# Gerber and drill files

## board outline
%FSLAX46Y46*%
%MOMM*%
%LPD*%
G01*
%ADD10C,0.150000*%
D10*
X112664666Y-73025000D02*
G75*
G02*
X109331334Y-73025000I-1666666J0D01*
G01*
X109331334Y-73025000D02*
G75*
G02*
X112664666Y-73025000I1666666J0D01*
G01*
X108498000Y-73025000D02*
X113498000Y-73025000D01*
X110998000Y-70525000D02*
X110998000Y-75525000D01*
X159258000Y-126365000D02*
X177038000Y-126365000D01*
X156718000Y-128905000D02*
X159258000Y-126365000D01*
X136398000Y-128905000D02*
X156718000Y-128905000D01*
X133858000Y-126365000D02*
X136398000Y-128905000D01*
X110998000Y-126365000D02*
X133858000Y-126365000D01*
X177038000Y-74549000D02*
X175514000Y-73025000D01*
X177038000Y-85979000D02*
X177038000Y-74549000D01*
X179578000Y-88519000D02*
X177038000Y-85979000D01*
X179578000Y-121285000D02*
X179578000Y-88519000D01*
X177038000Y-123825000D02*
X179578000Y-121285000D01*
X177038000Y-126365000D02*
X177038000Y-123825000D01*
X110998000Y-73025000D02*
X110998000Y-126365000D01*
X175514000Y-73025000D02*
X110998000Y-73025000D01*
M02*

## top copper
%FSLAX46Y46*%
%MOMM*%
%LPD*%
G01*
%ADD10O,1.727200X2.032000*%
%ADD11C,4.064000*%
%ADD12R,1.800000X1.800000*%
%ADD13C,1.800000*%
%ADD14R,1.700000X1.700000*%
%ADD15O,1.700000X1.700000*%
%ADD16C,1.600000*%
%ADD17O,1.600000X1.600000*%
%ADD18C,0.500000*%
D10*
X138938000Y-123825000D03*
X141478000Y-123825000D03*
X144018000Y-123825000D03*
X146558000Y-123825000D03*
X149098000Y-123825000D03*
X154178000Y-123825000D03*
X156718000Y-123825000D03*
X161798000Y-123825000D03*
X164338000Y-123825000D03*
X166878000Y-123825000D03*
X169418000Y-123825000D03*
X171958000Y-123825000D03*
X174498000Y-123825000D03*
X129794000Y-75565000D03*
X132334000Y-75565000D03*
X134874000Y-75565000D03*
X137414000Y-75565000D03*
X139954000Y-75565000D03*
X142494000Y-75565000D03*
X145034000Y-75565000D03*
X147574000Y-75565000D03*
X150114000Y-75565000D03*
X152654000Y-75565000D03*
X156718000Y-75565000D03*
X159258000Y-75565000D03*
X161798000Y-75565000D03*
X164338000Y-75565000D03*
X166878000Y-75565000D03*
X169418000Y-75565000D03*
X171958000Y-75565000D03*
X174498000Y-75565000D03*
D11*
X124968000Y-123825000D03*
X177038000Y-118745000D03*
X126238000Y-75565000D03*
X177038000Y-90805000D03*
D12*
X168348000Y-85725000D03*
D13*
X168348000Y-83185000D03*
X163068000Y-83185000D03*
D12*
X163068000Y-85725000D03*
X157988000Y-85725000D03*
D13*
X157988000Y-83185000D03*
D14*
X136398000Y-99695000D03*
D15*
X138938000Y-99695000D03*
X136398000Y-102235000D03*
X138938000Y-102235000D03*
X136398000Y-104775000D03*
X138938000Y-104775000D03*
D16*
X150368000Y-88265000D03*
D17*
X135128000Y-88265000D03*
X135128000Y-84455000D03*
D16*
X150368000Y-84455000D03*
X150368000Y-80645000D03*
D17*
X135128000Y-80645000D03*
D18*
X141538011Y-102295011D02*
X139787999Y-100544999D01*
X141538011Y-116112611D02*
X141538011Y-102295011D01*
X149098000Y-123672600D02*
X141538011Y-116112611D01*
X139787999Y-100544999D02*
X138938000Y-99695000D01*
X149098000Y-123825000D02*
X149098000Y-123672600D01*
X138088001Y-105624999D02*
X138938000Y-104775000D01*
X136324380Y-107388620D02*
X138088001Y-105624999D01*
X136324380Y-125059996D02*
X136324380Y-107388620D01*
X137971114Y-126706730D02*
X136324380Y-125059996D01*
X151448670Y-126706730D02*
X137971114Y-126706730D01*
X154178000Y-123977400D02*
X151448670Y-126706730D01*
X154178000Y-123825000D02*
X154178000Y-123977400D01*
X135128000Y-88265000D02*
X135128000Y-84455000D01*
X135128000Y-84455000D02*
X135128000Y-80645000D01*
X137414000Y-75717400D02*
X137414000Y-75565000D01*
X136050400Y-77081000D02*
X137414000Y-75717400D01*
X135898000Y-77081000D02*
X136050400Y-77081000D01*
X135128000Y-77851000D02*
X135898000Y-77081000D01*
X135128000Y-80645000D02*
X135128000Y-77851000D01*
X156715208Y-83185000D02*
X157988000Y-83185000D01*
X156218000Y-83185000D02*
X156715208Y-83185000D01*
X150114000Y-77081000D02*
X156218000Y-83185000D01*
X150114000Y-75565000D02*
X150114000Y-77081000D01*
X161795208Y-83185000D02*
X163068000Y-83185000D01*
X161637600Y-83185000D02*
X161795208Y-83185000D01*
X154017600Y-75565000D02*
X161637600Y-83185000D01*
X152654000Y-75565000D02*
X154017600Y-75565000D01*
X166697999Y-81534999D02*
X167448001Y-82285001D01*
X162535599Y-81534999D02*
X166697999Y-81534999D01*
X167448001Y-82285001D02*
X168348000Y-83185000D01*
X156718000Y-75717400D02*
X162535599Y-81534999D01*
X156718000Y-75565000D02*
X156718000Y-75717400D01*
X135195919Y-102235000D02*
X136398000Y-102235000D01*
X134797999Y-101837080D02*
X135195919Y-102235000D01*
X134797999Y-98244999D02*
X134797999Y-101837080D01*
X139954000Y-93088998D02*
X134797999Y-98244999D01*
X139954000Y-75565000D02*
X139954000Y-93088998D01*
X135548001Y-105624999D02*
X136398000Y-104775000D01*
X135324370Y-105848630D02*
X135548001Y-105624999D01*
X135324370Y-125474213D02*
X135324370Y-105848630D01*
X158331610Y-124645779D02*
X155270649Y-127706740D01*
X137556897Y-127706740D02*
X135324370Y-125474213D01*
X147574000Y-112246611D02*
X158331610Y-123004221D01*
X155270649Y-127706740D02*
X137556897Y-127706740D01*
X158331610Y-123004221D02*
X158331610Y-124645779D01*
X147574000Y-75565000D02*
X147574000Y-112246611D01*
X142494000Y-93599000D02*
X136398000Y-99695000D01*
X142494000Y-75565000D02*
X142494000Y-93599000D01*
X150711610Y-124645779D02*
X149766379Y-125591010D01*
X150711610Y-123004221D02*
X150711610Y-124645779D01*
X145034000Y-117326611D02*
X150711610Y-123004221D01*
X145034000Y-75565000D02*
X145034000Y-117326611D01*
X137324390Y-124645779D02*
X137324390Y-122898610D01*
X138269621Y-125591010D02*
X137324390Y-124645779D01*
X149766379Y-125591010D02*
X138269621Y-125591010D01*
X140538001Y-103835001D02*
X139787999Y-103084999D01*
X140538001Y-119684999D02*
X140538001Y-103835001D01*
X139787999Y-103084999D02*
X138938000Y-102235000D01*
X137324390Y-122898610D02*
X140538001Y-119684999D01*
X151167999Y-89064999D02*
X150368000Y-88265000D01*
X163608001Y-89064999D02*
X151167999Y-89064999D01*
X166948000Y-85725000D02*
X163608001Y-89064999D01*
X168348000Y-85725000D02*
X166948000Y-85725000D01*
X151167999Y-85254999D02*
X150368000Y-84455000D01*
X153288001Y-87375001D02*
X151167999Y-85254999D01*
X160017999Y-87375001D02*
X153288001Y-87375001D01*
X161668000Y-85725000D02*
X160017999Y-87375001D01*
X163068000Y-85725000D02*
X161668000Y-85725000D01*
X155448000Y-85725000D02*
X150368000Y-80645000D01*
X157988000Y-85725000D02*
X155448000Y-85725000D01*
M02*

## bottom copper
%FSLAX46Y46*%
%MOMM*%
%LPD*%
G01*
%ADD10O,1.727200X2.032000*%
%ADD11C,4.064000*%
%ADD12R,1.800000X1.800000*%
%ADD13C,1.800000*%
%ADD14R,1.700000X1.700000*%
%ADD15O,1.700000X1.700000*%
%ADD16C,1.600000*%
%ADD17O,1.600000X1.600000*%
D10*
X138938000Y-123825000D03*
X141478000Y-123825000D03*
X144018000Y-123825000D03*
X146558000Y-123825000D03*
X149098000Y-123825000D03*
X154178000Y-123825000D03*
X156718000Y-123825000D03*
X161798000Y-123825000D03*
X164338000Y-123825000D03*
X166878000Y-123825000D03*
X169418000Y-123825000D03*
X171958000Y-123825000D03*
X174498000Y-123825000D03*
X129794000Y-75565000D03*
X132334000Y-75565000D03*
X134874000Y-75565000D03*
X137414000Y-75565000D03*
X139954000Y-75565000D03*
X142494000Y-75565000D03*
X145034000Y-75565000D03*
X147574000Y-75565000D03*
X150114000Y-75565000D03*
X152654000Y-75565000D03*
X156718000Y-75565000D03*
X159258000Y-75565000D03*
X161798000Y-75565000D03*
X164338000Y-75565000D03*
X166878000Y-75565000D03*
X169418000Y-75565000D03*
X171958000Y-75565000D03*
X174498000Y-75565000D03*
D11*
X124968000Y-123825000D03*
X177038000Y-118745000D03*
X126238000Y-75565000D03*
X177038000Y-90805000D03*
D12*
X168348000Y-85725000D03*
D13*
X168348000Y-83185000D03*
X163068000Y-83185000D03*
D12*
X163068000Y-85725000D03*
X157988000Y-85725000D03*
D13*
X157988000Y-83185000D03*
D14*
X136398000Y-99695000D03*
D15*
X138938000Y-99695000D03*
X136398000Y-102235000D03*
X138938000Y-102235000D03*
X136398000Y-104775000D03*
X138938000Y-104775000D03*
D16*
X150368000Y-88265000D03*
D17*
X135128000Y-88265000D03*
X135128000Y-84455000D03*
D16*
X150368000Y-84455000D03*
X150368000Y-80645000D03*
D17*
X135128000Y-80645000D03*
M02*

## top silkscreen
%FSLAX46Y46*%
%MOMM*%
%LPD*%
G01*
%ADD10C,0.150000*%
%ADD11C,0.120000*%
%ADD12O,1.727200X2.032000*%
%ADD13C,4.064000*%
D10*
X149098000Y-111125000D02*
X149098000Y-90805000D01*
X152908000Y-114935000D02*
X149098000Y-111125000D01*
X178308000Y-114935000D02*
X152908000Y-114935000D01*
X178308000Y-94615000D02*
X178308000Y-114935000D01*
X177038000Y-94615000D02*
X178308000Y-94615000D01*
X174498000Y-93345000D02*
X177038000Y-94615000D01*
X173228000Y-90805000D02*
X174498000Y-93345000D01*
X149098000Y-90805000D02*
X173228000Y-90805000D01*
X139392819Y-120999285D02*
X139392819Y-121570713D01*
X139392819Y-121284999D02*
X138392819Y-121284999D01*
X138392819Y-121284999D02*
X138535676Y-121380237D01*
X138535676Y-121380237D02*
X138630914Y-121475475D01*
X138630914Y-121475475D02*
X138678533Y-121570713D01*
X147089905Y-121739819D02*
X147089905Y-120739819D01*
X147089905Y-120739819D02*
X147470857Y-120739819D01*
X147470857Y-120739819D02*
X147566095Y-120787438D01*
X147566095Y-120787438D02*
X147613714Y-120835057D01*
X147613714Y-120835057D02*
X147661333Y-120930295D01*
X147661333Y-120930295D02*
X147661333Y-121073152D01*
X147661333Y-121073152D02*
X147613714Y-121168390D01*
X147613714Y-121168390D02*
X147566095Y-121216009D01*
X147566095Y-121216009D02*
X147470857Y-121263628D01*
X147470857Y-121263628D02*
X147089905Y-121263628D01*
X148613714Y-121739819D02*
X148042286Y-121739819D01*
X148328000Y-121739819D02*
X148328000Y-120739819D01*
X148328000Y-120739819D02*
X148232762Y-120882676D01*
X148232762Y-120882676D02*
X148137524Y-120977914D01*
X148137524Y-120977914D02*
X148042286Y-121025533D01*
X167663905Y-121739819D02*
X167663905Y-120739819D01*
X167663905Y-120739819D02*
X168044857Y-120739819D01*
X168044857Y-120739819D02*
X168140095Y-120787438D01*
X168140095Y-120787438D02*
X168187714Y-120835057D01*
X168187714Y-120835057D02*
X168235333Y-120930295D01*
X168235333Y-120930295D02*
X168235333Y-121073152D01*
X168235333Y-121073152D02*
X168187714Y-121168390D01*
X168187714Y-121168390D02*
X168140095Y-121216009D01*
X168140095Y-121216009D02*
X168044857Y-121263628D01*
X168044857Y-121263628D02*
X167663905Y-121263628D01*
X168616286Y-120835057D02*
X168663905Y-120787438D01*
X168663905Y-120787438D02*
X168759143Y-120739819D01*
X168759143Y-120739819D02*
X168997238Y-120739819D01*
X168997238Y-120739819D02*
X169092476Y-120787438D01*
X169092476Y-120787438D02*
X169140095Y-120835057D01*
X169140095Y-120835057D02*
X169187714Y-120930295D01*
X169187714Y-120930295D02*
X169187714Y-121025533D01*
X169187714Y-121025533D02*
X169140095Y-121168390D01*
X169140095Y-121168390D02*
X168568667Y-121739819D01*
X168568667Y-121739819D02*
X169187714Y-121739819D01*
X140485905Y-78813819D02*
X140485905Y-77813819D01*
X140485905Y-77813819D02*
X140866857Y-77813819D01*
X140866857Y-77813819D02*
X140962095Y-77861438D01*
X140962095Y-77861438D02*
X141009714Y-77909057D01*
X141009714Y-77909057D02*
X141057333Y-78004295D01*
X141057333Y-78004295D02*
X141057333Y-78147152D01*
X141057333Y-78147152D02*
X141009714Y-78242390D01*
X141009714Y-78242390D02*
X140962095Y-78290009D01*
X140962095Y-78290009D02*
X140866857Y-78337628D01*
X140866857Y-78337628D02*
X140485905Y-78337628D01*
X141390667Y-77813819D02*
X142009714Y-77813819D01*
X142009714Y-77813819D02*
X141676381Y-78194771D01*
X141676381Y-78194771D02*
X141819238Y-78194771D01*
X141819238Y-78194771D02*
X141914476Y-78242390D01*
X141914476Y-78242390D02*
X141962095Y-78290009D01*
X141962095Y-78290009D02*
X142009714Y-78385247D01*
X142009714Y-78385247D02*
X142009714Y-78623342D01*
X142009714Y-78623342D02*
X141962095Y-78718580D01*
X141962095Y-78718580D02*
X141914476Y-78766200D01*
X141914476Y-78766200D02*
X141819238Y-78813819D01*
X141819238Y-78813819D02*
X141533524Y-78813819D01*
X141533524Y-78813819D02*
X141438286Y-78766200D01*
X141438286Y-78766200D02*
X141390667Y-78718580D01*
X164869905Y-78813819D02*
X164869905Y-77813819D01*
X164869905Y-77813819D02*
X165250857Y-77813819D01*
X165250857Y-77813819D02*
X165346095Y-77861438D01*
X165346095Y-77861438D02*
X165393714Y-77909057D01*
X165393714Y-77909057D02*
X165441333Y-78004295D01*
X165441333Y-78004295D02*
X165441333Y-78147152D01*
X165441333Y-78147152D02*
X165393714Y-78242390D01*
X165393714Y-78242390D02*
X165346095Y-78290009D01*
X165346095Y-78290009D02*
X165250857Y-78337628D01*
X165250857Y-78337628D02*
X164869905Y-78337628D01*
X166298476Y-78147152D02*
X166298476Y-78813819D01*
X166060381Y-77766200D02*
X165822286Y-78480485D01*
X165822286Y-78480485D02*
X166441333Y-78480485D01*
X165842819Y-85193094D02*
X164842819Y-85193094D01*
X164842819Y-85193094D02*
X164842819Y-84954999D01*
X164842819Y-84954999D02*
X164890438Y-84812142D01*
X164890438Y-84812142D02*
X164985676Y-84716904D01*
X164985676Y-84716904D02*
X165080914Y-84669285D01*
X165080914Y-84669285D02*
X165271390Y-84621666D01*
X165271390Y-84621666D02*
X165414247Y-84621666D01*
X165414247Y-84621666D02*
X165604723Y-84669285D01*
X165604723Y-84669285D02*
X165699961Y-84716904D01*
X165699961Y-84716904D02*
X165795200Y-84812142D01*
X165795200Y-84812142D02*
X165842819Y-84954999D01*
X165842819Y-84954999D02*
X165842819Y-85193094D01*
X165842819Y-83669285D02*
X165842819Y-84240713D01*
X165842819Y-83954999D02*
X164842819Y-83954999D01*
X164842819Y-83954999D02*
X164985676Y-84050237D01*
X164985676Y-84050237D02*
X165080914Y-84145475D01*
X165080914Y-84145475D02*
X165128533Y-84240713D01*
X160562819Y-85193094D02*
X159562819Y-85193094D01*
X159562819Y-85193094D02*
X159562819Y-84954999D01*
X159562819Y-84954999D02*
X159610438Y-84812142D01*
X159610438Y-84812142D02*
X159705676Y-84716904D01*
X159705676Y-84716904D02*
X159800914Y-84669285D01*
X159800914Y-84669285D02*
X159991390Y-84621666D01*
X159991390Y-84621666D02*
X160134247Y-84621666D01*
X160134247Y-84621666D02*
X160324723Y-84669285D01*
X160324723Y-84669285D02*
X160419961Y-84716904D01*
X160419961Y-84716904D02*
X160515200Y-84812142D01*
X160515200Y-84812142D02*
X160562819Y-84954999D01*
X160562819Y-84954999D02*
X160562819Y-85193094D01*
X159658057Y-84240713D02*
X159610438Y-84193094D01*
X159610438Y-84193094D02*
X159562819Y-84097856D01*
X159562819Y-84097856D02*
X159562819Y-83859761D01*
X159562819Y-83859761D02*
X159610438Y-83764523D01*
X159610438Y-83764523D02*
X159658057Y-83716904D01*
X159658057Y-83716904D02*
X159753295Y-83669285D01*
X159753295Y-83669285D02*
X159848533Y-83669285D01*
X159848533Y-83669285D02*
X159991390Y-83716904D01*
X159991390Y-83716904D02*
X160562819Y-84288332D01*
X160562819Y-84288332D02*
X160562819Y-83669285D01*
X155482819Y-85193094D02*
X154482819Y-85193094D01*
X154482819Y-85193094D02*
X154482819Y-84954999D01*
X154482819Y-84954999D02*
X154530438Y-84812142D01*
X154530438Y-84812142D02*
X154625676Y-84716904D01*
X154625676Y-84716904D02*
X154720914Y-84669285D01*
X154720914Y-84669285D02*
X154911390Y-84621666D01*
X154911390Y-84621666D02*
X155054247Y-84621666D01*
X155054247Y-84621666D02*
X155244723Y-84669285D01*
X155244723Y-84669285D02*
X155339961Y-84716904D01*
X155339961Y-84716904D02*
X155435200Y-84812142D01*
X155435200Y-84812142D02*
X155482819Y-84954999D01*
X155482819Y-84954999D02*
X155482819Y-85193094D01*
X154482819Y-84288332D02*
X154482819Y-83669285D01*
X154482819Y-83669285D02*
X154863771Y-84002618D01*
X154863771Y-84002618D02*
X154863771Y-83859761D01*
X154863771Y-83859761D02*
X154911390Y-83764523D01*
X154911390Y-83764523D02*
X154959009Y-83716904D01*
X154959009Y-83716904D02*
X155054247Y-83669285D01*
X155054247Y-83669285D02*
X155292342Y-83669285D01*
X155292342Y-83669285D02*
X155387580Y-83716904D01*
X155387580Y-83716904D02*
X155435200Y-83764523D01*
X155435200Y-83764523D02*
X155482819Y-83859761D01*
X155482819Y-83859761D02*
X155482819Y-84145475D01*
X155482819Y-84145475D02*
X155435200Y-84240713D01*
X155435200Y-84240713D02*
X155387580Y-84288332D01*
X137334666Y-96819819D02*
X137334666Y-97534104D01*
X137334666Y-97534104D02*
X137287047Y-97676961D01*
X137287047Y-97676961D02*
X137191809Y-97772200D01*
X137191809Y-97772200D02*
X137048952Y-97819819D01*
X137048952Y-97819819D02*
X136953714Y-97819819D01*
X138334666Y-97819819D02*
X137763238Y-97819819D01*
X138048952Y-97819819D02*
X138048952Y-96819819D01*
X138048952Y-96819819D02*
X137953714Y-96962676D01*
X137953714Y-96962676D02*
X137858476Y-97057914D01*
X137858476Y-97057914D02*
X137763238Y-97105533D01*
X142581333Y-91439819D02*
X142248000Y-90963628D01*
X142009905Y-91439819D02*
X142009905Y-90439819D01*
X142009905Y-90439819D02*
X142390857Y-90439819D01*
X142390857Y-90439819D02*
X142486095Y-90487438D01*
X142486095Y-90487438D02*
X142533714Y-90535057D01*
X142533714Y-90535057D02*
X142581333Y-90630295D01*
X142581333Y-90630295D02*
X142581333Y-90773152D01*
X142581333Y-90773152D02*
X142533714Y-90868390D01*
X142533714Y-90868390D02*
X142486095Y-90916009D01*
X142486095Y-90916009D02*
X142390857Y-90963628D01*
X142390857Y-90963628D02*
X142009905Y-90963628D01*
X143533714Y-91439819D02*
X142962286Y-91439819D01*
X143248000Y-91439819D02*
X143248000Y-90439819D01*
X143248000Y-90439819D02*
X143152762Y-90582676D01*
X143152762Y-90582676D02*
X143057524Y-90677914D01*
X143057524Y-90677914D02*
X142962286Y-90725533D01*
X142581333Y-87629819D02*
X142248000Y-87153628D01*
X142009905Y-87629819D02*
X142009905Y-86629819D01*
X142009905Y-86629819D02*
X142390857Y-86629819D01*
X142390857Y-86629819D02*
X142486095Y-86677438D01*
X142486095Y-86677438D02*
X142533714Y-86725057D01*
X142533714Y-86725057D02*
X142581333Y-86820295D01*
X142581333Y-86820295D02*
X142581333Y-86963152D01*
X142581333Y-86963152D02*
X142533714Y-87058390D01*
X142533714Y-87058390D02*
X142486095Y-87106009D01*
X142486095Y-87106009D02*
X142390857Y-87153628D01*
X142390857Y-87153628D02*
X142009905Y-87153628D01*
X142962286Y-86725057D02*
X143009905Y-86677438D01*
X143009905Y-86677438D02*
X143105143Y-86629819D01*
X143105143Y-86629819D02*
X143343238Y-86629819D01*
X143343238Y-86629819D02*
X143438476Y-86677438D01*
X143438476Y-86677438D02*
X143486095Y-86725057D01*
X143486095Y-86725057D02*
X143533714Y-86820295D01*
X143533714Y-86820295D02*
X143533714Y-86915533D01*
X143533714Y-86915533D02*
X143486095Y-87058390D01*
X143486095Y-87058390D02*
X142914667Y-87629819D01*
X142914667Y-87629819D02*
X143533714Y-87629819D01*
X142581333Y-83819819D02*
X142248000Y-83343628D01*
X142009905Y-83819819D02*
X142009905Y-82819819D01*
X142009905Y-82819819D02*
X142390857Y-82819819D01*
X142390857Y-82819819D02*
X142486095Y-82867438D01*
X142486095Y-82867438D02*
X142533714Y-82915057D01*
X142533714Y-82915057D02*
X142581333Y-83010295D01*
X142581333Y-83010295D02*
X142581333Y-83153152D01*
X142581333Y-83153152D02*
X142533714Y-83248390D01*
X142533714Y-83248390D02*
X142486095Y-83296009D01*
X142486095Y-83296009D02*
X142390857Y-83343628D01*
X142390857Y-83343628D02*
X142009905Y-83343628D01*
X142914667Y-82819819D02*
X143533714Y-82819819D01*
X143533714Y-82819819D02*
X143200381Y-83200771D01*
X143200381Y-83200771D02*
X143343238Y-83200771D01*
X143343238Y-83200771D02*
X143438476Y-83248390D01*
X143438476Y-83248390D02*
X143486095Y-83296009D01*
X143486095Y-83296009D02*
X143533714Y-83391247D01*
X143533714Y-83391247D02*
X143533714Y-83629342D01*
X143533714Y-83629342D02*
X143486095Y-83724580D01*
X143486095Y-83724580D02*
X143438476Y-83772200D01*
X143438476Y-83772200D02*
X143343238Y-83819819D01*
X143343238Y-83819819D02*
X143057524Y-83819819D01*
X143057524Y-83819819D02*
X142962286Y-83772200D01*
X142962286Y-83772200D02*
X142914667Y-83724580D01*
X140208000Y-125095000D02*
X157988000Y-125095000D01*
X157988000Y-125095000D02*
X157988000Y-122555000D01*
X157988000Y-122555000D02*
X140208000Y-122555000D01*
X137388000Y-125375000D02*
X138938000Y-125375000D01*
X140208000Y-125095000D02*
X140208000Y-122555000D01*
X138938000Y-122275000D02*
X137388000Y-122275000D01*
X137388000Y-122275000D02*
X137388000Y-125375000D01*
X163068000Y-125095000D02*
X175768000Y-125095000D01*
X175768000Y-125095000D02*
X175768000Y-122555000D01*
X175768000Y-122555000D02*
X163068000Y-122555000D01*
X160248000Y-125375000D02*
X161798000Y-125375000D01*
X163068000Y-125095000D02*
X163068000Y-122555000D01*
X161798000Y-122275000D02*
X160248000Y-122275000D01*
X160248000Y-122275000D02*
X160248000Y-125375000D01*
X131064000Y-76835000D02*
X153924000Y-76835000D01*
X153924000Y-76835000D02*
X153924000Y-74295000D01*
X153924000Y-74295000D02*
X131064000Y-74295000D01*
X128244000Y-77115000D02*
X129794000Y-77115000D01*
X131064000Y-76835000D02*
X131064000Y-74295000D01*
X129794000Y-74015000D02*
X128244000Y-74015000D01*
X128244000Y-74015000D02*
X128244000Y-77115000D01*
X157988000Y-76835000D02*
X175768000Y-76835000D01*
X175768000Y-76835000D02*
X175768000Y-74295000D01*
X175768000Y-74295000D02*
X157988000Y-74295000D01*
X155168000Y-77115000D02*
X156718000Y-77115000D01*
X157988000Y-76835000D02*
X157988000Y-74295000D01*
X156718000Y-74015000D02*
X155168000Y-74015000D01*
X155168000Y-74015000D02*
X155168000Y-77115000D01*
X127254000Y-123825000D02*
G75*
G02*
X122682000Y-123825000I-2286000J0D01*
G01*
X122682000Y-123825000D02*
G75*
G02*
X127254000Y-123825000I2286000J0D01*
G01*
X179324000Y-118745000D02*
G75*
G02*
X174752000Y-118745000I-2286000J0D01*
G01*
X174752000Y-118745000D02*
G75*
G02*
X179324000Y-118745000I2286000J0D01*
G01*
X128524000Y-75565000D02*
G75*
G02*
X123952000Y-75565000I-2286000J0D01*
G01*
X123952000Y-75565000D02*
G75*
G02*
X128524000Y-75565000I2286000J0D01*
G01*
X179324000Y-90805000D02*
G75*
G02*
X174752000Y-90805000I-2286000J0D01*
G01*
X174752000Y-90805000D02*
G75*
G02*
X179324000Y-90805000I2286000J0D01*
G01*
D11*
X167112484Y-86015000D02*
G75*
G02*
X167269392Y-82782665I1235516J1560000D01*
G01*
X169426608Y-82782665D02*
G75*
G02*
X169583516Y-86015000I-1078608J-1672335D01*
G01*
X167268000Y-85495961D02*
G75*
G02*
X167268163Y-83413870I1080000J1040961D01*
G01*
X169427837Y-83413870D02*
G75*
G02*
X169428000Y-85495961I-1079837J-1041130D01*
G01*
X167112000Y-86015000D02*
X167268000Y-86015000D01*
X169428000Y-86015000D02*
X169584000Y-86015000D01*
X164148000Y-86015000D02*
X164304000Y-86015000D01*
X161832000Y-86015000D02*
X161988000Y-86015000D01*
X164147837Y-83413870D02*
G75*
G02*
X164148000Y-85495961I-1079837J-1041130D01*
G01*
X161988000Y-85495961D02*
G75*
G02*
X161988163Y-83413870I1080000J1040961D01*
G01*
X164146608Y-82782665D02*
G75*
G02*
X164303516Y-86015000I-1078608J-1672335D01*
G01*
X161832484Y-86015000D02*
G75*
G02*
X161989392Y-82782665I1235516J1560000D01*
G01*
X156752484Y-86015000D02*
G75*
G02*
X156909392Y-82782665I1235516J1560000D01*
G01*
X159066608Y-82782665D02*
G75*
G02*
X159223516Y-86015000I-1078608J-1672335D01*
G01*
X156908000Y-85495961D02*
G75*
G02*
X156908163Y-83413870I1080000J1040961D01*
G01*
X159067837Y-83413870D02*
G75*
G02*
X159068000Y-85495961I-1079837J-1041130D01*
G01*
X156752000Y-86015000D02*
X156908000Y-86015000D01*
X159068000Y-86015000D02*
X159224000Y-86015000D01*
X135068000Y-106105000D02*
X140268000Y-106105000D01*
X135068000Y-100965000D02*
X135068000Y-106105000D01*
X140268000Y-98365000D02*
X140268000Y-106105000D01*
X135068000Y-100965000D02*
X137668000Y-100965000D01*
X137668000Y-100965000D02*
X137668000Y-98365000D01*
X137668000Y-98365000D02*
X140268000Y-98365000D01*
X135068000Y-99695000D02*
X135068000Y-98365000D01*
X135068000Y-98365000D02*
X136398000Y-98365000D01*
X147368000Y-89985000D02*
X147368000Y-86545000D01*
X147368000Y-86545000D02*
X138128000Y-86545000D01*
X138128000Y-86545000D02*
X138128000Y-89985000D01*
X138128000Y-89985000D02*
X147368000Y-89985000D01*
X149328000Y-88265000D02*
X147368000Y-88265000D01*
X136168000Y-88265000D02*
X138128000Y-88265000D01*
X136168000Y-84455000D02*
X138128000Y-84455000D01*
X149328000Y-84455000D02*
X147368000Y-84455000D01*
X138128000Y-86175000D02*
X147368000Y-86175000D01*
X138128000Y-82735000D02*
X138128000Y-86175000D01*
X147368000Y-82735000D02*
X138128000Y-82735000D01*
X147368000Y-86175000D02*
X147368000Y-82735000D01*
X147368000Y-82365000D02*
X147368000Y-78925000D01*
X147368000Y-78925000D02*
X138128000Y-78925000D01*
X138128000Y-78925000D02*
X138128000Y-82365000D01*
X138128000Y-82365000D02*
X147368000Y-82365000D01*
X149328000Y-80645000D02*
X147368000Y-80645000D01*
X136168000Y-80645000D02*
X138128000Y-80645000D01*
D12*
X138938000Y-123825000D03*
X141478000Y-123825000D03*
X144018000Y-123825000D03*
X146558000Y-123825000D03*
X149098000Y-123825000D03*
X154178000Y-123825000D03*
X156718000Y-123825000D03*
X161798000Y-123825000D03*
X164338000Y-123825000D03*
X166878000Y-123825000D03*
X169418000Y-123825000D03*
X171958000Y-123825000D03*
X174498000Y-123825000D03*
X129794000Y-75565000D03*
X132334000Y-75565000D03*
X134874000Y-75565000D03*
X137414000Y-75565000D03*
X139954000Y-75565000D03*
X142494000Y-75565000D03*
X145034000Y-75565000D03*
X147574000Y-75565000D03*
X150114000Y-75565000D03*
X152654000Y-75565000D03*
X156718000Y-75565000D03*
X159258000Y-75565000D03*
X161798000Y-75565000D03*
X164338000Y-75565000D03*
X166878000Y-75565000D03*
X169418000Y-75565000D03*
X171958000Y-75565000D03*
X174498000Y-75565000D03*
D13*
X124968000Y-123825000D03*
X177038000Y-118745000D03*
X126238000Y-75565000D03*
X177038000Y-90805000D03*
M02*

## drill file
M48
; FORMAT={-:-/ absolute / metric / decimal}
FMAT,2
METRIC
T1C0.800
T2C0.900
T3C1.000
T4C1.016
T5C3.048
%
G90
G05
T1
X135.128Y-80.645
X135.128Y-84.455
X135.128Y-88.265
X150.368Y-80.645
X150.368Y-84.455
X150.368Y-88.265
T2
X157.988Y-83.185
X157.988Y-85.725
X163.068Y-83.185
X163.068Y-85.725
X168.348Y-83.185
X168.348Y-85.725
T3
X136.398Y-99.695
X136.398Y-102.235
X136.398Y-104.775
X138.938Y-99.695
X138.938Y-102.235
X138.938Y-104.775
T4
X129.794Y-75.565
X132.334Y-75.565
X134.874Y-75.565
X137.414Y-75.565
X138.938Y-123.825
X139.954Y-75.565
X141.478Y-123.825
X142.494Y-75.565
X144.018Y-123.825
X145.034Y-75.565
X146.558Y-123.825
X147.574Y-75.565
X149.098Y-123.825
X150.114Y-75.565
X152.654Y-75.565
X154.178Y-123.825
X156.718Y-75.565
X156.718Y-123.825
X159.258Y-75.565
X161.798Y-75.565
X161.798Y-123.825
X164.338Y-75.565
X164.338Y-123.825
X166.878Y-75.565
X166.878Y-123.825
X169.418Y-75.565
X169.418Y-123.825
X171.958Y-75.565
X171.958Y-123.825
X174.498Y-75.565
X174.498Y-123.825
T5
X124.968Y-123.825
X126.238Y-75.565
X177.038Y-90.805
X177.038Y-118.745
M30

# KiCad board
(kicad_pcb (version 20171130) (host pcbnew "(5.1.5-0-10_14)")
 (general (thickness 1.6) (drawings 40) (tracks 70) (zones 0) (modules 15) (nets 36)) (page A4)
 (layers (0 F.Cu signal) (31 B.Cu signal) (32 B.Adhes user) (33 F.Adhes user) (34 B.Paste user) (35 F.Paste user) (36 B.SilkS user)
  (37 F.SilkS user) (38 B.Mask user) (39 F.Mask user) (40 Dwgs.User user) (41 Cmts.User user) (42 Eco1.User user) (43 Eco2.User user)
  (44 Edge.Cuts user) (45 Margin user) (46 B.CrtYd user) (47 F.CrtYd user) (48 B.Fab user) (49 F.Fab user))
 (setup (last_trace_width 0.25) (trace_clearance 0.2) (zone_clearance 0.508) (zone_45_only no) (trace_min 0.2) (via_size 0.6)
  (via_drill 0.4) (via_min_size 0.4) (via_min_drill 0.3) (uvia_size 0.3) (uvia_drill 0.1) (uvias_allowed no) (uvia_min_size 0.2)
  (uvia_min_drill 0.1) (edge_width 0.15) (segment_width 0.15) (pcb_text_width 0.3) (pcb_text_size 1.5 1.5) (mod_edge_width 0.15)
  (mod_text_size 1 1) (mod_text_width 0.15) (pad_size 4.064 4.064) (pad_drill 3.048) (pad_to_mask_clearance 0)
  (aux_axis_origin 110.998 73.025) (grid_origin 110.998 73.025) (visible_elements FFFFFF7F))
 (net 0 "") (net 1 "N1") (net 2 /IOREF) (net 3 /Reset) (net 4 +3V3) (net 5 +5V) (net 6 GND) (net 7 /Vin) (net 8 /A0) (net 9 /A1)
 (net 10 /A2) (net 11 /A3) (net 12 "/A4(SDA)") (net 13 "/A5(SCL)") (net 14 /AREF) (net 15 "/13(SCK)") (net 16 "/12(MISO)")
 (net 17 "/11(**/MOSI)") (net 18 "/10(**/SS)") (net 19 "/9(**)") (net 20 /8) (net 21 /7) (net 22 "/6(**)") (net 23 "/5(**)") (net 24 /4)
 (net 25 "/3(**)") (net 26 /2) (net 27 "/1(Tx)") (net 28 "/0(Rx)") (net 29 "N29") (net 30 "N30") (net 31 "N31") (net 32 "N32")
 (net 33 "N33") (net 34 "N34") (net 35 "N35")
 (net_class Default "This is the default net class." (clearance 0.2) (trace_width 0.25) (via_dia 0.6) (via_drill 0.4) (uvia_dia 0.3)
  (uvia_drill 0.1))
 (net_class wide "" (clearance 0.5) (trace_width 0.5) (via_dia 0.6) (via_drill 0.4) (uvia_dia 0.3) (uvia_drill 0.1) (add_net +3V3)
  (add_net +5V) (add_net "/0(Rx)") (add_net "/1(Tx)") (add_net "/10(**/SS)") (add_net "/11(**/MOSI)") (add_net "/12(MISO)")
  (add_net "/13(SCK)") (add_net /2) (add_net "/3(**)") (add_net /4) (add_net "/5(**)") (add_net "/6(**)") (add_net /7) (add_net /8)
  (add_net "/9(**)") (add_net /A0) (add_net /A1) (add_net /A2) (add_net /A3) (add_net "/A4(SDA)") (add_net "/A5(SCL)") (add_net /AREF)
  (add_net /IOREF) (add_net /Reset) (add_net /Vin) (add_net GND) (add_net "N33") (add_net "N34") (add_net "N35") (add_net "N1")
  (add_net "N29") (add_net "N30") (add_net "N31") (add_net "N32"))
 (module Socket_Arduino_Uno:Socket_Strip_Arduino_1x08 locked (layer F.Cu) (at 138.938 123.825)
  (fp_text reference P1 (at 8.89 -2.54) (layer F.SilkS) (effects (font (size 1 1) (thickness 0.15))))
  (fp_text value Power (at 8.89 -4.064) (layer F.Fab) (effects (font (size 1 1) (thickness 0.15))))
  (fp_line (start 1.27 1.27) (end 19.05 1.27) (layer F.SilkS) (width 0.15))
  (fp_line (start 19.05 1.27) (end 19.05 -1.27) (layer F.SilkS) (width 0.15))
  (fp_line (start 19.05 -1.27) (end 1.27 -1.27) (layer F.SilkS) (width 0.15))
  (fp_line (start -1.55 1.55) (end 0 1.55) (layer F.SilkS) (width 0.15))
  (fp_line (start 1.27 1.27) (end 1.27 -1.27) (layer F.SilkS) (width 0.15))
  (fp_line (start 0 -1.55) (end -1.55 -1.55) (layer F.SilkS) (width 0.15))
  (fp_line (start -1.55 -1.55) (end -1.55 1.55) (layer F.SilkS) (width 0.15))
  (pad 1 thru_hole oval (at 0 0) (size 1.7272 2.032) (drill 1.016) (layers *.Cu *.Mask F.SilkS) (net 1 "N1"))
  (pad 2 thru_hole oval (at 2.54 0) (size 1.7272 2.032) (drill 1.016) (layers *.Cu *.Mask F.SilkS) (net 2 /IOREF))
  (pad 3 thru_hole oval (at 5.08 0) (size 1.7272 2.032) (drill 1.016) (layers *.Cu *.Mask F.SilkS) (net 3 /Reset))
  (pad 4 thru_hole oval (at 7.62 0) (size 1.7272 2.032) (drill 1.016) (layers *.Cu *.Mask F.SilkS) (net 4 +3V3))
  (pad 5 thru_hole oval (at 10.16 0) (size 1.7272 2.032) (drill 1.016) (layers *.Cu *.Mask F.SilkS) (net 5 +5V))
  (pad 6 connect oval (at 12.7 0) (size 1.7272 2.032) (layers Dwgs.User) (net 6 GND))
  (pad 7 thru_hole oval (at 15.24 0) (size 1.7272 2.032) (drill 1.016) (layers *.Cu *.Mask F.SilkS) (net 6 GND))
  (pad 8 thru_hole oval (at 17.78 0) (size 1.7272 2.032) (drill 1.016) (layers *.Cu *.Mask F.SilkS) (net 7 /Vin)))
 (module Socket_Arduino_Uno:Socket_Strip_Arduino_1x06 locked (layer F.Cu) (at 161.798 123.825)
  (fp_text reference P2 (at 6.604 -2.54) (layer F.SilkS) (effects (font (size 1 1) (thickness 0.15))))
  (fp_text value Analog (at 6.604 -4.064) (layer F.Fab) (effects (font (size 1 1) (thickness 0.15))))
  (fp_line (start 1.27 1.27) (end 13.97 1.27) (layer F.SilkS) (width 0.15))
  (fp_line (start 13.97 1.27) (end 13.97 -1.27) (layer F.SilkS) (width 0.15))
  (fp_line (start 13.97 -1.27) (end 1.27 -1.27) (layer F.SilkS) (width 0.15))
  (fp_line (start -1.55 1.55) (end 0 1.55) (layer F.SilkS) (width 0.15))
  (fp_line (start 1.27 1.27) (end 1.27 -1.27) (layer F.SilkS) (width 0.15))
  (fp_line (start 0 -1.55) (end -1.55 -1.55) (layer F.SilkS) (width 0.15))
  (fp_line (start -1.55 -1.55) (end -1.55 1.55) (layer F.SilkS) (width 0.15))
  (pad 1 thru_hole oval (at 0 0) (size 1.7272 2.032) (drill 1.016) (layers *.Cu *.Mask F.SilkS) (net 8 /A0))
  (pad 2 thru_hole oval (at 2.54 0) (size 1.7272 2.032) (drill 1.016) (layers *.Cu *.Mask F.SilkS) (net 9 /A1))
  (pad 3 thru_hole oval (at 5.08 0) (size 1.7272 2.032) (drill 1.016) (layers *.Cu *.Mask F.SilkS) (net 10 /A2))
  (pad 4 thru_hole oval (at 7.62 0) (size 1.7272 2.032) (drill 1.016) (layers *.Cu *.Mask F.SilkS) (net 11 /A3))
  (pad 5 thru_hole oval (at 10.16 0) (size 1.7272 2.032) (drill 1.016) (layers *.Cu *.Mask F.SilkS) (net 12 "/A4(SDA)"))
  (pad 6 thru_hole oval (at 12.7 0) (size 1.7272 2.032) (drill 1.016) (layers *.Cu *.Mask F.SilkS) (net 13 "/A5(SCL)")))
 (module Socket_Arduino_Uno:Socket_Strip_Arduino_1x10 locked (layer F.Cu) (at 129.794 75.565)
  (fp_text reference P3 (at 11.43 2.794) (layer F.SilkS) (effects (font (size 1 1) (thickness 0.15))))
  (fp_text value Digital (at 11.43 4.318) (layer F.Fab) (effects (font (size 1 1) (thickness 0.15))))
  (fp_line (start 1.27 1.27) (end 24.13 1.27) (layer F.SilkS) (width 0.15))
  (fp_line (start 24.13 1.27) (end 24.13 -1.27) (layer F.SilkS) (width 0.15))
  (fp_line (start 24.13 -1.27) (end 1.27 -1.27) (layer F.SilkS) (width 0.15))
  (fp_line (start -1.55 1.55) (end 0 1.55) (layer F.SilkS) (width 0.15))
  (fp_line (start 1.27 1.27) (end 1.27 -1.27) (layer F.SilkS) (width 0.15))
  (fp_line (start 0 -1.55) (end -1.55 -1.55) (layer F.SilkS) (width 0.15))
  (fp_line (start -1.55 -1.55) (end -1.55 1.55) (layer F.SilkS) (width 0.15))
  (pad 1 thru_hole oval (at 0 0) (size 1.7272 2.032) (drill 1.016) (layers *.Cu *.Mask F.SilkS) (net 13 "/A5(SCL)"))
  (pad 2 thru_hole oval (at 2.54 0) (size 1.7272 2.032) (drill 1.016) (layers *.Cu *.Mask F.SilkS) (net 12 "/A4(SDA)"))
  (pad 3 thru_hole oval (at 5.08 0) (size 1.7272 2.032) (drill 1.016) (layers *.Cu *.Mask F.SilkS) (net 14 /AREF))
  (pad 4 thru_hole oval (at 7.62 0) (size 1.7272 2.032) (drill 1.016) (layers *.Cu *.Mask F.SilkS) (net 6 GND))
  (pad 5 thru_hole oval (at 10.16 0) (size 1.7272 2.032) (drill 1.016) (layers *.Cu *.Mask F.SilkS) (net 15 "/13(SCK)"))
  (pad 6 thru_hole oval (at 12.7 0) (size 1.7272 2.032) (drill 1.016) (layers *.Cu *.Mask F.SilkS) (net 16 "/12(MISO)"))
  (pad 7 thru_hole oval (at 15.24 0) (size 1.7272 2.032) (drill 1.016) (layers *.Cu *.Mask F.SilkS) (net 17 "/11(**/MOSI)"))
  (pad 8 thru_hole oval (at 17.78 0) (size 1.7272 2.032) (drill 1.016) (layers *.Cu *.Mask F.SilkS) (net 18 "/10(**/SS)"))
  (pad 9 thru_hole oval (at 20.32 0) (size 1.7272 2.032) (drill 1.016) (layers *.Cu *.Mask F.SilkS) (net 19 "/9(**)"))
  (pad 10 thru_hole oval (at 22.86 0) (size 1.7272 2.032) (drill 1.016) (layers *.Cu *.Mask F.SilkS) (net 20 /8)))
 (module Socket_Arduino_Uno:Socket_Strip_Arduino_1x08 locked (layer F.Cu) (at 156.718 75.565)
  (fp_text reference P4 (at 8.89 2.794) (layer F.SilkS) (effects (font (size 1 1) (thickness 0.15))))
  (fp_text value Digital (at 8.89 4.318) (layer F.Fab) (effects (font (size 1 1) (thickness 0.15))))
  (fp_line (start 1.27 1.27) (end 19.05 1.27) (layer F.SilkS) (width 0.15))
  (fp_line (start 19.05 1.27) (end 19.05 -1.27) (layer F.SilkS) (width 0.15))
  (fp_line (start 19.05 -1.27) (end 1.27 -1.27) (layer F.SilkS) (width 0.15))
  (fp_line (start -1.55 1.55) (end 0 1.55) (layer F.SilkS) (width 0.15))
  (fp_line (start 1.27 1.27) (end 1.27 -1.27) (layer F.SilkS) (width 0.15))
  (fp_line (start 0 -1.55) (end -1.55 -1.55) (layer F.SilkS) (width 0.15))
  (fp_line (start -1.55 -1.55) (end -1.55 1.55) (layer F.SilkS) (width 0.15))
  (pad 1 thru_hole oval (at 0 0) (size 1.7272 2.032) (drill 1.016) (layers *.Cu *.Mask F.SilkS) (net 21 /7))
  (pad 2 thru_hole oval (at 2.54 0) (size 1.7272 2.032) (drill 1.016) (layers *.Cu *.Mask F.SilkS) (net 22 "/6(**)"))
  (pad 3 thru_hole oval (at 5.08 0) (size 1.7272 2.032) (drill 1.016) (layers *.Cu *.Mask F.SilkS) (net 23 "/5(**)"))
  (pad 4 thru_hole oval (at 7.62 0) (size 1.7272 2.032) (drill 1.016) (layers *.Cu *.Mask F.SilkS) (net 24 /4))
  (pad 5 thru_hole oval (at 10.16 0) (size 1.7272 2.032) (drill 1.016) (layers *.Cu *.Mask F.SilkS) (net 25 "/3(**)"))
  (pad 6 thru_hole oval (at 12.7 0) (size 1.7272 2.032) (drill 1.016) (layers *.Cu *.Mask F.SilkS) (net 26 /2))
  (pad 7 thru_hole oval (at 15.24 0) (size 1.7272 2.032) (drill 1.016) (layers *.Cu *.Mask F.SilkS) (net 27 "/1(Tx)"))
  (pad 8 thru_hole oval (at 17.78 0) (size 1.7272 2.032) (drill 1.016) (layers *.Cu *.Mask F.SilkS) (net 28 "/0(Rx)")))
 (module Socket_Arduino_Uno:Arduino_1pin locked (layer F.Cu) (at 124.968 123.825)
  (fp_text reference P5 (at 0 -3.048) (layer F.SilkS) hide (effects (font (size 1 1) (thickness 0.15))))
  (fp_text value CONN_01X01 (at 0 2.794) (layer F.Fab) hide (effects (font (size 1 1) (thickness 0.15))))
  (fp_circle (center 0 0) (end 0 -2.286) (layer F.SilkS) (width 0.15))
  (pad 1 thru_hole circle (at 0 0) (size 4.064 4.064) (drill 3.048) (layers *.Cu *.Mask F.SilkS) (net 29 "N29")))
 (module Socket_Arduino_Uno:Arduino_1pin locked (layer F.Cu) (at 177.038 118.745)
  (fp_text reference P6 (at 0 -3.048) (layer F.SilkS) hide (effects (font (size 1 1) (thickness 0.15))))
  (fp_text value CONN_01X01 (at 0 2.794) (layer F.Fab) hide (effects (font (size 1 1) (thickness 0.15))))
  (fp_circle (center 0 0) (end 0 -2.286) (layer F.SilkS) (width 0.15))
  (pad 1 thru_hole circle (at 0 0) (size 4.064 4.064) (drill 3.048) (layers *.Cu *.Mask F.SilkS) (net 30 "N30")))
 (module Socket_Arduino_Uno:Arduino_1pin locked (layer F.Cu) (at 126.238 75.565)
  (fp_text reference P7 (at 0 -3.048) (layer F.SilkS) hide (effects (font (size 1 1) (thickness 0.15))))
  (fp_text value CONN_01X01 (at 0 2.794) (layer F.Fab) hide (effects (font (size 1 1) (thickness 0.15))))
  (fp_circle (center 0 0) (end 0 -2.286) (layer F.SilkS) (width 0.15))
  (pad 1 thru_hole circle (at 0 0) (size 4.064 4.064) (drill 3.048) (layers *.Cu *.Mask F.SilkS) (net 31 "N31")))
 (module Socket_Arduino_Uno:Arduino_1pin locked (layer F.Cu) (at 177.038 90.805)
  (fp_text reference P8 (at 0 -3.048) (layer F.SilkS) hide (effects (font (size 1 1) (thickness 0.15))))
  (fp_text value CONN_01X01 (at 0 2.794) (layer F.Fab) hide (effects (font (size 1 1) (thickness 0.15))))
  (fp_circle (center 0 0) (end 0 -2.286) (layer F.SilkS) (width 0.15))
  (pad 1 thru_hole circle (at 0 0) (size 4.064 4.064) (drill 3.048) (layers *.Cu *.Mask F.SilkS) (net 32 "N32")))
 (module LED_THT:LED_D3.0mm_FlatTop (layer F.Cu) (at 168.348 85.725 90)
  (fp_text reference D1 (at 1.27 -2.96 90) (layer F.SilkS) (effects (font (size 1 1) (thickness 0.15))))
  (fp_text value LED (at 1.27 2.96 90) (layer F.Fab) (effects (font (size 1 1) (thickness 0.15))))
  (fp_arc (start 1.27 0) (end -0.29 -1.235516) (angle 108.8) (layer F.SilkS) (width 0.12))
  (fp_arc (start 1.27 0) (end -0.29 1.235516) (angle -108.8) (layer F.SilkS) (width 0.12))
  (fp_arc (start 1.27 0) (end 0.229039 -1.08) (angle 87.9) (layer F.SilkS) (width 0.12))
  (fp_arc (start 1.27 0) (end 0.229039 1.08) (angle -87.9) (layer F.SilkS) (width 0.12))
  (fp_line (start -0.29 -1.236) (end -0.29 -1.08) (layer F.SilkS) (width 0.12))
  (fp_line (start -0.29 1.08) (end -0.29 1.236) (layer F.SilkS) (width 0.12))
  (pad 1 thru_hole rect (at 0 0 90) (size 1.8 1.8) (drill 0.9) (layers *.Cu *.Mask) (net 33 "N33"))
  (pad 2 thru_hole circle (at 2.54 0 90) (size 1.8 1.8) (drill 0.9) (layers *.Cu *.Mask) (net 21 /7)))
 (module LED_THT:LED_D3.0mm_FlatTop (layer F.Cu) (at 163.068 85.725 90)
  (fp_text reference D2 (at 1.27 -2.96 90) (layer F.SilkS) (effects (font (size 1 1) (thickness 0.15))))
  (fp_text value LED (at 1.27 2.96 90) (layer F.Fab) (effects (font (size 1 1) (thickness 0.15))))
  (fp_line (start -0.29 1.08) (end -0.29 1.236) (layer F.SilkS) (width 0.12))
  (fp_line (start -0.29 -1.236) (end -0.29 -1.08) (layer F.SilkS) (width 0.12))
  (fp_arc (start 1.27 0) (end 0.229039 1.08) (angle -87.9) (layer F.SilkS) (width 0.12))
  (fp_arc (start 1.27 0) (end 0.229039 -1.08) (angle 87.9) (layer F.SilkS) (width 0.12))
  (fp_arc (start 1.27 0) (end -0.29 1.235516) (angle -108.8) (layer F.SilkS) (width 0.12))
  (fp_arc (start 1.27 0) (end -0.29 -1.235516) (angle 108.8) (layer F.SilkS) (width 0.12))
  (pad 2 thru_hole circle (at 2.54 0 90) (size 1.8 1.8) (drill 0.9) (layers *.Cu *.Mask) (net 20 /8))
  (pad 1 thru_hole rect (at 0 0 90) (size 1.8 1.8) (drill 0.9) (layers *.Cu *.Mask) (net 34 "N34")))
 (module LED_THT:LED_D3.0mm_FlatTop (layer F.Cu) (at 157.988 85.725 90)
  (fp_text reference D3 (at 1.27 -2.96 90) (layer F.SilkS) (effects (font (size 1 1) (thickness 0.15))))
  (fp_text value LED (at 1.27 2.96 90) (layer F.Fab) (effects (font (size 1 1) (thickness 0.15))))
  (fp_arc (start 1.27 0) (end -0.29 -1.235516) (angle 108.8) (layer F.SilkS) (width 0.12))
  (fp_arc (start 1.27 0) (end -0.29 1.235516) (angle -108.8) (layer F.SilkS) (width 0.12))
  (fp_arc (start 1.27 0) (end 0.229039 -1.08) (angle 87.9) (layer F.SilkS) (width 0.12))
  (fp_arc (start 1.27 0) (end 0.229039 1.08) (angle -87.9) (layer F.SilkS) (width 0.12))
  (fp_line (start -0.29 -1.236) (end -0.29 -1.08) (layer F.SilkS) (width 0.12))
  (fp_line (start -0.29 1.08) (end -0.29 1.236) (layer F.SilkS) (width 0.12))
  (pad 1 thru_hole rect (at 0 0 90) (size 1.8 1.8) (drill 0.9) (layers *.Cu *.Mask) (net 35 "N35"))
  (pad 2 thru_hole circle (at 2.54 0 90) (size 1.8 1.8) (drill 0.9) (layers *.Cu *.Mask) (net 19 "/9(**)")))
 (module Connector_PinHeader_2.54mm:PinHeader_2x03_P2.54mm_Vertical (layer F.Cu) (at 136.398 99.695)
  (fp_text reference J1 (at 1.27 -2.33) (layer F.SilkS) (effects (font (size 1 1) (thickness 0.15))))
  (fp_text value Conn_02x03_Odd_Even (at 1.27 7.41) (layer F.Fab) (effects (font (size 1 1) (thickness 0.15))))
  (fp_line (start -1.33 6.41) (end 3.87 6.41) (layer F.SilkS) (width 0.12))
  (fp_line (start -1.33 1.27) (end -1.33 6.41) (layer F.SilkS) (width 0.12))
  (fp_line (start 3.87 -1.33) (end 3.87 6.41) (layer F.SilkS) (width 0.12))
  (fp_line (start -1.33 1.27) (end 1.27 1.27) (layer F.SilkS) (width 0.12))
  (fp_line (start 1.27 1.27) (end 1.27 -1.33) (layer F.SilkS) (width 0.12))
  (fp_line (start 1.27 -1.33) (end 3.87 -1.33) (layer F.SilkS) (width 0.12))
  (fp_line (start -1.33 0) (end -1.33 -1.33) (layer F.SilkS) (width 0.12))
  (fp_line (start -1.33 -1.33) (end 0 -1.33) (layer F.SilkS) (width 0.12))
  (pad 1 thru_hole rect (at 0 0) (size 1.7 1.7) (drill 1) (layers *.Cu *.Mask) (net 16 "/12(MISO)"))
  (pad 2 thru_hole oval (at 2.54 0) (size 1.7 1.7) (drill 1) (layers *.Cu *.Mask) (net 5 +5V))
  (pad 3 thru_hole oval (at 0 2.54) (size 1.7 1.7) (drill 1) (layers *.Cu *.Mask) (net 15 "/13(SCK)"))
  (pad 4 thru_hole oval (at 2.54 2.54) (size 1.7 1.7) (drill 1) (layers *.Cu *.Mask) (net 17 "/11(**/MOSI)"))
  (pad 5 thru_hole oval (at 0 5.08) (size 1.7 1.7) (drill 1) (layers *.Cu *.Mask) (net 18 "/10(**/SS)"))
  (pad 6 thru_hole oval (at 2.54 5.08) (size 1.7 1.7) (drill 1) (layers *.Cu *.Mask) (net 6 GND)))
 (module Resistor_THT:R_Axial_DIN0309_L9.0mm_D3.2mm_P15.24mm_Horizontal (layer F.Cu) (at 150.368 88.265 180)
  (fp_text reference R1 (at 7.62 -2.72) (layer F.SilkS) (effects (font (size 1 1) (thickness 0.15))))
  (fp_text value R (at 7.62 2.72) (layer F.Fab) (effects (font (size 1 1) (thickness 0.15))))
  (fp_line (start 3 -1.72) (end 3 1.72) (layer F.SilkS) (width 0.12))
  (fp_line (start 3 1.72) (end 12.24 1.72) (layer F.SilkS) (width 0.12))
  (fp_line (start 12.24 1.72) (end 12.24 -1.72) (layer F.SilkS) (width 0.12))
  (fp_line (start 12.24 -1.72) (end 3 -1.72) (layer F.SilkS) (width 0.12))
  (fp_line (start 1.04 0) (end 3 0) (layer F.SilkS) (width 0.12))
  (fp_line (start 14.2 0) (end 12.24 0) (layer F.SilkS) (width 0.12))
  (pad 1 thru_hole circle (at 0 0 180) (size 1.6 1.6) (drill 0.8) (layers *.Cu *.Mask) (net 33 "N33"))
  (pad 2 thru_hole oval (at 15.24 0 180) (size 1.6 1.6) (drill 0.8) (layers *.Cu *.Mask) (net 6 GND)))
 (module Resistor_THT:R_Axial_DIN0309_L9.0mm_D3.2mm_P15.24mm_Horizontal (layer F.Cu) (at 150.368 84.455 180)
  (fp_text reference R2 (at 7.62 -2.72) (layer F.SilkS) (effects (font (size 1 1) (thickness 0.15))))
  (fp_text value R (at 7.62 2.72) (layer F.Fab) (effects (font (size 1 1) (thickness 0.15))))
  (fp_line (start 14.2 0) (end 12.24 0) (layer F.SilkS) (width 0.12))
  (fp_line (start 1.04 0) (end 3 0) (layer F.SilkS) (width 0.12))
  (fp_line (start 12.24 -1.72) (end 3 -1.72) (layer F.SilkS) (width 0.12))
  (fp_line (start 12.24 1.72) (end 12.24 -1.72) (layer F.SilkS) (width 0.12))
  (fp_line (start 3 1.72) (end 12.24 1.72) (layer F.SilkS) (width 0.12))
  (fp_line (start 3 -1.72) (end 3 1.72) (layer F.SilkS) (width 0.12))
  (pad 2 thru_hole oval (at 15.24 0 180) (size 1.6 1.6) (drill 0.8) (layers *.Cu *.Mask) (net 6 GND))
  (pad 1 thru_hole circle (at 0 0 180) (size 1.6 1.6) (drill 0.8) (layers *.Cu *.Mask) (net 34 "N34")))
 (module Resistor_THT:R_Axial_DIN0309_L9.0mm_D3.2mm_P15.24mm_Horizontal (layer F.Cu) (at 150.368 80.645 180)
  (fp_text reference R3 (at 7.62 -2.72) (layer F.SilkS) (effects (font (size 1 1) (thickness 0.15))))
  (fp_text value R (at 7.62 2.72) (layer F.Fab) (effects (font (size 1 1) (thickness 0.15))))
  (fp_line (start 3 -1.72) (end 3 1.72) (layer F.SilkS) (width 0.12))
  (fp_line (start 3 1.72) (end 12.24 1.72) (layer F.SilkS) (width 0.12))
  (fp_line (start 12.24 1.72) (end 12.24 -1.72) (layer F.SilkS) (width 0.12))
  (fp_line (start 12.24 -1.72) (end 3 -1.72) (layer F.SilkS) (width 0.12))
  (fp_line (start 1.04 0) (end 3 0) (layer F.SilkS) (width 0.12))
  (fp_line (start 14.2 0) (end 12.24 0) (layer F.SilkS) (width 0.12))
  (pad 1 thru_hole circle (at 0 0 180) (size 1.6 1.6) (drill 0.8) (layers *.Cu *.Mask) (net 35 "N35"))
  (pad 2 thru_hole oval (at 15.24 0 180) (size 1.6 1.6) (drill 0.8) (layers *.Cu *.Mask) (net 6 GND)))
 (gr_line (start 149.098 111.125) (end 149.098 90.805) (layer F.SilkS) (width 0.15))
 (gr_line (start 152.908 114.935) (end 149.098 111.125) (layer F.SilkS) (width 0.15))
 (gr_line (start 178.308 114.935) (end 152.908 114.935) (layer F.SilkS) (width 0.15))
 (gr_line (start 178.308 94.615) (end 178.308 114.935) (layer F.SilkS) (width 0.15))
 (gr_line (start 177.038 94.615) (end 178.308 94.615) (layer F.SilkS) (width 0.15))
 (gr_line (start 174.498 93.345) (end 177.038 94.615) (layer F.SilkS) (width 0.15))
 (gr_line (start 173.228 90.805) (end 174.498 93.345) (layer F.SilkS) (width 0.15))
 (gr_line (start 149.098 90.805) (end 173.228 90.805) (layer F.SilkS) (width 0.15))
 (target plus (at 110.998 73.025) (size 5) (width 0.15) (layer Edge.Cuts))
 (gr_line (start 159.258 126.365) (end 177.038 126.365) (layer Edge.Cuts) (width 0.15))
 (gr_line (start 156.718 128.905) (end 159.258 126.365) (layer Edge.Cuts) (width 0.15))
 (gr_line (start 136.398 128.905) (end 156.718 128.905) (layer Edge.Cuts) (width 0.15))
 (gr_line (start 133.858 126.365) (end 136.398 128.905) (layer Edge.Cuts) (width 0.15))
 (gr_line (start 110.998 126.365) (end 133.858 126.365) (layer Edge.Cuts) (width 0.15))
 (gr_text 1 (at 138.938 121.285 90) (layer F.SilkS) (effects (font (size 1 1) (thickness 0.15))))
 (gr_line (start 177.038 74.549) (end 175.514 73.025) (angle 90) (layer Edge.Cuts) (width 0.15))
 (gr_line (start 177.038 85.979) (end 177.038 74.549) (angle 90) (layer Edge.Cuts) (width 0.15))
 (gr_line (start 179.578 88.519) (end 177.038 85.979) (angle 90) (layer Edge.Cuts) (width 0.15))
 (gr_line (start 179.578 121.285) (end 179.578 88.519) (angle 90) (layer Edge.Cuts) (width 0.15))
 (gr_line (start 177.038 123.825) (end 179.578 121.285) (angle 90) (layer Edge.Cuts) (width 0.15))
 (gr_line (start 177.038 126.365) (end 177.038 123.825) (angle 90) (layer Edge.Cuts) (width 0.15))
 (gr_line (start 110.998 73.025) (end 110.998 126.365) (angle 90) (layer Edge.Cuts) (width 0.15))
 (gr_line (start 175.514 73.025) (end 110.998 73.025) (angle 90) (layer Edge.Cuts) (width 0.15))
 (segment (start 141.538011 102.295011) (end 139.787999 100.544999) (width 0.5) (layer F.Cu) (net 5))
 (segment (start 141.538011 116.112611) (end 141.538011 102.295011) (width 0.5) (layer F.Cu) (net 5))
 (segment (start 149.098 123.6726) (end 141.538011 116.112611) (width 0.5) (layer F.Cu) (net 5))
 (segment (start 139.787999 100.544999) (end 138.938 99.695) (width 0.5) (layer F.Cu) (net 5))
 (segment (start 149.098 123.825) (end 149.098 123.6726) (width 0.5) (layer F.Cu) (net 5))
 (segment (start 138.088001 105.624999) (end 138.938 104.775) (width 0.5) (layer F.Cu) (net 6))
 (segment (start 136.32438 107.38862) (end 138.088001 105.624999) (width 0.5) (layer F.Cu) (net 6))
 (segment (start 136.32438 125.059996) (end 136.32438 107.38862) (width 0.5) (layer F.Cu) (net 6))
 (segment (start 137.971114 126.70673) (end 136.32438 125.059996) (width 0.5) (layer F.Cu) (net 6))
 (segment (start 151.44867 126.70673) (end 137.971114 126.70673) (width 0.5) (layer F.Cu) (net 6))
 (segment (start 154.178 123.9774) (end 151.44867 126.70673) (width 0.5) (layer F.Cu) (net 6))
 (segment (start 154.178 123.825) (end 154.178 123.9774) (width 0.5) (layer F.Cu) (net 6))
 (segment (start 135.128 88.265) (end 135.128 84.455) (width 0.5) (layer F.Cu) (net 6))
 (segment (start 135.128 84.455) (end 135.128 80.645) (width 0.5) (layer F.Cu) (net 6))
 (segment (start 137.414 75.7174) (end 137.414 75.565) (width 0.5) (layer F.Cu) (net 6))
 (segment (start 136.0504 77.081) (end 137.414 75.7174) (width 0.5) (layer F.Cu) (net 6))
 (segment (start 135.898 77.081) (end 136.0504 77.081) (width 0.5) (layer F.Cu) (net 6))
 (segment (start 135.128 77.851) (end 135.898 77.081) (width 0.5) (layer F.Cu) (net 6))
 (segment (start 135.128 80.645) (end 135.128 77.851) (width 0.5) (layer F.Cu) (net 6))
 (segment (start 156.715208 83.185) (end 157.988 83.185) (width 0.5) (layer F.Cu) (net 19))
 (segment (start 156.218 83.185) (end 156.715208 83.185) (width 0.5) (layer F.Cu) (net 19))
 (segment (start 150.114 77.081) (end 156.218 83.185) (width 0.5) (layer F.Cu) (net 19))
 (segment (start 150.114 75.565) (end 150.114 77.081) (width 0.5) (layer F.Cu) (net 19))
 (segment (start 161.795208 83.185) (end 163.068 83.185) (width 0.5) (layer F.Cu) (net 20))
 (segment (start 161.6376 83.185) (end 161.795208 83.185) (width 0.5) (layer F.Cu) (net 20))
 (segment (start 154.0176 75.565) (end 161.6376 83.185) (width 0.5) (layer F.Cu) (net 20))
 (segment (start 152.654 75.565) (end 154.0176 75.565) (width 0.5) (layer F.Cu) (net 20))
 (segment (start 166.697999 81.534999) (end 167.448001 82.285001) (width 0.5) (layer F.Cu) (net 21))
 (segment (start 162.535599 81.534999) (end 166.697999 81.534999) (width 0.5) (layer F.Cu) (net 21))
 (segment (start 167.448001 82.285001) (end 168.348 83.185) (width 0.5) (layer F.Cu) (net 21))
 (segment (start 156.718 75.7174) (end 162.535599 81.534999) (width 0.5) (layer F.Cu) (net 21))
 (segment (start 156.718 75.565) (end 156.718 75.7174) (width 0.5) (layer F.Cu) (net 21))
 (segment (start 135.195919 102.235) (end 136.398 102.235) (width 0.5) (layer F.Cu) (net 15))
 (segment (start 134.797999 101.83708) (end 135.195919 102.235) (width 0.5) (layer F.Cu) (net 15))
 (segment (start 134.797999 98.244999) (end 134.797999 101.83708) (width 0.5) (layer F.Cu) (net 15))
 (segment (start 139.954 93.088998) (end 134.797999 98.244999) (width 0.5) (layer F.Cu) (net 15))
 (segment (start 139.954 75.565) (end 139.954 93.088998) (width 0.5) (layer F.Cu) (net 15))
 (segment (start 135.548001 105.624999) (end 136.398 104.775) (width 0.5) (layer F.Cu) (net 18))
 (segment (start 135.32437 105.84863) (end 135.548001 105.624999) (width 0.5) (layer F.Cu) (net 18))
 (segment (start 135.32437 125.474213) (end 135.32437 105.84863) (width 0.5) (layer F.Cu) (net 18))
 (segment (start 158.33161 124.645779) (end 155.270649 127.70674) (width 0.5) (layer F.Cu) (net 18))
 (segment (start 137.556897 127.70674) (end 135.32437 125.474213) (width 0.5) (layer F.Cu) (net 18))
 (segment (start 147.574 112.246611) (end 158.33161 123.004221) (width 0.5) (layer F.Cu) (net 18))
 (segment (start 155.270649 127.70674) (end 137.556897 127.70674) (width 0.5) (layer F.Cu) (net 18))
 (segment (start 158.33161 123.004221) (end 158.33161 124.645779) (width 0.5) (layer F.Cu) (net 18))
 (segment (start 147.574 75.565) (end 147.574 112.246611) (width 0.5) (layer F.Cu) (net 18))
 (segment (start 142.494 93.599) (end 136.398 99.695) (width 0.5) (layer F.Cu) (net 16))
 (segment (start 142.494 75.565) (end 142.494 93.599) (width 0.5) (layer F.Cu) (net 16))
 (segment (start 150.71161 124.645779) (end 149.766379 125.59101) (width 0.5) (layer F.Cu) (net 17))
 (segment (start 150.71161 123.004221) (end 150.71161 124.645779) (width 0.5) (layer F.Cu) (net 17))
 (segment (start 145.034 117.326611) (end 150.71161 123.004221) (width 0.5) (layer F.Cu) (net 17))
 (segment (start 145.034 75.565) (end 145.034 117.326611) (width 0.5) (layer F.Cu) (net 17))
 (segment (start 137.32439 124.645779) (end 137.32439 122.89861) (width 0.5) (layer F.Cu) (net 17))
 (segment (start 138.269621 125.59101) (end 137.32439 124.645779) (width 0.5) (layer F.Cu) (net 17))
 (segment (start 149.766379 125.59101) (end 138.269621 125.59101) (width 0.5) (layer F.Cu) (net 17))
 (segment (start 140.538001 103.835001) (end 139.787999 103.084999) (width 0.5) (layer F.Cu) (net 17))
 (segment (start 140.538001 119.684999) (end 140.538001 103.835001) (width 0.5) (layer F.Cu) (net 17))
 (segment (start 139.787999 103.084999) (end 138.938 102.235) (width 0.5) (layer F.Cu) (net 17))
 (segment (start 137.32439 122.89861) (end 140.538001 119.684999) (width 0.5) (layer F.Cu) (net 17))
 (segment (start 151.167999 89.064999) (end 150.368 88.265) (width 0.5) (layer F.Cu) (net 33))
 (segment (start 163.608001 89.064999) (end 151.167999 89.064999) (width 0.5) (layer F.Cu) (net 33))
 (segment (start 166.948 85.725) (end 163.608001 89.064999) (width 0.5) (layer F.Cu) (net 33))
 (segment (start 168.348 85.725) (end 166.948 85.725) (width 0.5) (layer F.Cu) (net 33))
 (segment (start 151.167999 85.254999) (end 150.368 84.455) (width 0.5) (layer F.Cu) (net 34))
 (segment (start 153.288001 87.375001) (end 151.167999 85.254999) (width 0.5) (layer F.Cu) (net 34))
 (segment (start 160.017999 87.375001) (end 153.288001 87.375001) (width 0.5) (layer F.Cu) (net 34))
 (segment (start 161.668 85.725) (end 160.017999 87.375001) (width 0.5) (layer F.Cu) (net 34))
 (segment (start 163.068 85.725) (end 161.668 85.725) (width 0.5) (layer F.Cu) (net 34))
 (segment (start 155.448 85.725) (end 150.368 80.645) (width 0.5) (layer F.Cu) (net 35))
 (segment (start 157.988 85.725) (end 155.448 85.725) (width 0.5) (layer F.Cu) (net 35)))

